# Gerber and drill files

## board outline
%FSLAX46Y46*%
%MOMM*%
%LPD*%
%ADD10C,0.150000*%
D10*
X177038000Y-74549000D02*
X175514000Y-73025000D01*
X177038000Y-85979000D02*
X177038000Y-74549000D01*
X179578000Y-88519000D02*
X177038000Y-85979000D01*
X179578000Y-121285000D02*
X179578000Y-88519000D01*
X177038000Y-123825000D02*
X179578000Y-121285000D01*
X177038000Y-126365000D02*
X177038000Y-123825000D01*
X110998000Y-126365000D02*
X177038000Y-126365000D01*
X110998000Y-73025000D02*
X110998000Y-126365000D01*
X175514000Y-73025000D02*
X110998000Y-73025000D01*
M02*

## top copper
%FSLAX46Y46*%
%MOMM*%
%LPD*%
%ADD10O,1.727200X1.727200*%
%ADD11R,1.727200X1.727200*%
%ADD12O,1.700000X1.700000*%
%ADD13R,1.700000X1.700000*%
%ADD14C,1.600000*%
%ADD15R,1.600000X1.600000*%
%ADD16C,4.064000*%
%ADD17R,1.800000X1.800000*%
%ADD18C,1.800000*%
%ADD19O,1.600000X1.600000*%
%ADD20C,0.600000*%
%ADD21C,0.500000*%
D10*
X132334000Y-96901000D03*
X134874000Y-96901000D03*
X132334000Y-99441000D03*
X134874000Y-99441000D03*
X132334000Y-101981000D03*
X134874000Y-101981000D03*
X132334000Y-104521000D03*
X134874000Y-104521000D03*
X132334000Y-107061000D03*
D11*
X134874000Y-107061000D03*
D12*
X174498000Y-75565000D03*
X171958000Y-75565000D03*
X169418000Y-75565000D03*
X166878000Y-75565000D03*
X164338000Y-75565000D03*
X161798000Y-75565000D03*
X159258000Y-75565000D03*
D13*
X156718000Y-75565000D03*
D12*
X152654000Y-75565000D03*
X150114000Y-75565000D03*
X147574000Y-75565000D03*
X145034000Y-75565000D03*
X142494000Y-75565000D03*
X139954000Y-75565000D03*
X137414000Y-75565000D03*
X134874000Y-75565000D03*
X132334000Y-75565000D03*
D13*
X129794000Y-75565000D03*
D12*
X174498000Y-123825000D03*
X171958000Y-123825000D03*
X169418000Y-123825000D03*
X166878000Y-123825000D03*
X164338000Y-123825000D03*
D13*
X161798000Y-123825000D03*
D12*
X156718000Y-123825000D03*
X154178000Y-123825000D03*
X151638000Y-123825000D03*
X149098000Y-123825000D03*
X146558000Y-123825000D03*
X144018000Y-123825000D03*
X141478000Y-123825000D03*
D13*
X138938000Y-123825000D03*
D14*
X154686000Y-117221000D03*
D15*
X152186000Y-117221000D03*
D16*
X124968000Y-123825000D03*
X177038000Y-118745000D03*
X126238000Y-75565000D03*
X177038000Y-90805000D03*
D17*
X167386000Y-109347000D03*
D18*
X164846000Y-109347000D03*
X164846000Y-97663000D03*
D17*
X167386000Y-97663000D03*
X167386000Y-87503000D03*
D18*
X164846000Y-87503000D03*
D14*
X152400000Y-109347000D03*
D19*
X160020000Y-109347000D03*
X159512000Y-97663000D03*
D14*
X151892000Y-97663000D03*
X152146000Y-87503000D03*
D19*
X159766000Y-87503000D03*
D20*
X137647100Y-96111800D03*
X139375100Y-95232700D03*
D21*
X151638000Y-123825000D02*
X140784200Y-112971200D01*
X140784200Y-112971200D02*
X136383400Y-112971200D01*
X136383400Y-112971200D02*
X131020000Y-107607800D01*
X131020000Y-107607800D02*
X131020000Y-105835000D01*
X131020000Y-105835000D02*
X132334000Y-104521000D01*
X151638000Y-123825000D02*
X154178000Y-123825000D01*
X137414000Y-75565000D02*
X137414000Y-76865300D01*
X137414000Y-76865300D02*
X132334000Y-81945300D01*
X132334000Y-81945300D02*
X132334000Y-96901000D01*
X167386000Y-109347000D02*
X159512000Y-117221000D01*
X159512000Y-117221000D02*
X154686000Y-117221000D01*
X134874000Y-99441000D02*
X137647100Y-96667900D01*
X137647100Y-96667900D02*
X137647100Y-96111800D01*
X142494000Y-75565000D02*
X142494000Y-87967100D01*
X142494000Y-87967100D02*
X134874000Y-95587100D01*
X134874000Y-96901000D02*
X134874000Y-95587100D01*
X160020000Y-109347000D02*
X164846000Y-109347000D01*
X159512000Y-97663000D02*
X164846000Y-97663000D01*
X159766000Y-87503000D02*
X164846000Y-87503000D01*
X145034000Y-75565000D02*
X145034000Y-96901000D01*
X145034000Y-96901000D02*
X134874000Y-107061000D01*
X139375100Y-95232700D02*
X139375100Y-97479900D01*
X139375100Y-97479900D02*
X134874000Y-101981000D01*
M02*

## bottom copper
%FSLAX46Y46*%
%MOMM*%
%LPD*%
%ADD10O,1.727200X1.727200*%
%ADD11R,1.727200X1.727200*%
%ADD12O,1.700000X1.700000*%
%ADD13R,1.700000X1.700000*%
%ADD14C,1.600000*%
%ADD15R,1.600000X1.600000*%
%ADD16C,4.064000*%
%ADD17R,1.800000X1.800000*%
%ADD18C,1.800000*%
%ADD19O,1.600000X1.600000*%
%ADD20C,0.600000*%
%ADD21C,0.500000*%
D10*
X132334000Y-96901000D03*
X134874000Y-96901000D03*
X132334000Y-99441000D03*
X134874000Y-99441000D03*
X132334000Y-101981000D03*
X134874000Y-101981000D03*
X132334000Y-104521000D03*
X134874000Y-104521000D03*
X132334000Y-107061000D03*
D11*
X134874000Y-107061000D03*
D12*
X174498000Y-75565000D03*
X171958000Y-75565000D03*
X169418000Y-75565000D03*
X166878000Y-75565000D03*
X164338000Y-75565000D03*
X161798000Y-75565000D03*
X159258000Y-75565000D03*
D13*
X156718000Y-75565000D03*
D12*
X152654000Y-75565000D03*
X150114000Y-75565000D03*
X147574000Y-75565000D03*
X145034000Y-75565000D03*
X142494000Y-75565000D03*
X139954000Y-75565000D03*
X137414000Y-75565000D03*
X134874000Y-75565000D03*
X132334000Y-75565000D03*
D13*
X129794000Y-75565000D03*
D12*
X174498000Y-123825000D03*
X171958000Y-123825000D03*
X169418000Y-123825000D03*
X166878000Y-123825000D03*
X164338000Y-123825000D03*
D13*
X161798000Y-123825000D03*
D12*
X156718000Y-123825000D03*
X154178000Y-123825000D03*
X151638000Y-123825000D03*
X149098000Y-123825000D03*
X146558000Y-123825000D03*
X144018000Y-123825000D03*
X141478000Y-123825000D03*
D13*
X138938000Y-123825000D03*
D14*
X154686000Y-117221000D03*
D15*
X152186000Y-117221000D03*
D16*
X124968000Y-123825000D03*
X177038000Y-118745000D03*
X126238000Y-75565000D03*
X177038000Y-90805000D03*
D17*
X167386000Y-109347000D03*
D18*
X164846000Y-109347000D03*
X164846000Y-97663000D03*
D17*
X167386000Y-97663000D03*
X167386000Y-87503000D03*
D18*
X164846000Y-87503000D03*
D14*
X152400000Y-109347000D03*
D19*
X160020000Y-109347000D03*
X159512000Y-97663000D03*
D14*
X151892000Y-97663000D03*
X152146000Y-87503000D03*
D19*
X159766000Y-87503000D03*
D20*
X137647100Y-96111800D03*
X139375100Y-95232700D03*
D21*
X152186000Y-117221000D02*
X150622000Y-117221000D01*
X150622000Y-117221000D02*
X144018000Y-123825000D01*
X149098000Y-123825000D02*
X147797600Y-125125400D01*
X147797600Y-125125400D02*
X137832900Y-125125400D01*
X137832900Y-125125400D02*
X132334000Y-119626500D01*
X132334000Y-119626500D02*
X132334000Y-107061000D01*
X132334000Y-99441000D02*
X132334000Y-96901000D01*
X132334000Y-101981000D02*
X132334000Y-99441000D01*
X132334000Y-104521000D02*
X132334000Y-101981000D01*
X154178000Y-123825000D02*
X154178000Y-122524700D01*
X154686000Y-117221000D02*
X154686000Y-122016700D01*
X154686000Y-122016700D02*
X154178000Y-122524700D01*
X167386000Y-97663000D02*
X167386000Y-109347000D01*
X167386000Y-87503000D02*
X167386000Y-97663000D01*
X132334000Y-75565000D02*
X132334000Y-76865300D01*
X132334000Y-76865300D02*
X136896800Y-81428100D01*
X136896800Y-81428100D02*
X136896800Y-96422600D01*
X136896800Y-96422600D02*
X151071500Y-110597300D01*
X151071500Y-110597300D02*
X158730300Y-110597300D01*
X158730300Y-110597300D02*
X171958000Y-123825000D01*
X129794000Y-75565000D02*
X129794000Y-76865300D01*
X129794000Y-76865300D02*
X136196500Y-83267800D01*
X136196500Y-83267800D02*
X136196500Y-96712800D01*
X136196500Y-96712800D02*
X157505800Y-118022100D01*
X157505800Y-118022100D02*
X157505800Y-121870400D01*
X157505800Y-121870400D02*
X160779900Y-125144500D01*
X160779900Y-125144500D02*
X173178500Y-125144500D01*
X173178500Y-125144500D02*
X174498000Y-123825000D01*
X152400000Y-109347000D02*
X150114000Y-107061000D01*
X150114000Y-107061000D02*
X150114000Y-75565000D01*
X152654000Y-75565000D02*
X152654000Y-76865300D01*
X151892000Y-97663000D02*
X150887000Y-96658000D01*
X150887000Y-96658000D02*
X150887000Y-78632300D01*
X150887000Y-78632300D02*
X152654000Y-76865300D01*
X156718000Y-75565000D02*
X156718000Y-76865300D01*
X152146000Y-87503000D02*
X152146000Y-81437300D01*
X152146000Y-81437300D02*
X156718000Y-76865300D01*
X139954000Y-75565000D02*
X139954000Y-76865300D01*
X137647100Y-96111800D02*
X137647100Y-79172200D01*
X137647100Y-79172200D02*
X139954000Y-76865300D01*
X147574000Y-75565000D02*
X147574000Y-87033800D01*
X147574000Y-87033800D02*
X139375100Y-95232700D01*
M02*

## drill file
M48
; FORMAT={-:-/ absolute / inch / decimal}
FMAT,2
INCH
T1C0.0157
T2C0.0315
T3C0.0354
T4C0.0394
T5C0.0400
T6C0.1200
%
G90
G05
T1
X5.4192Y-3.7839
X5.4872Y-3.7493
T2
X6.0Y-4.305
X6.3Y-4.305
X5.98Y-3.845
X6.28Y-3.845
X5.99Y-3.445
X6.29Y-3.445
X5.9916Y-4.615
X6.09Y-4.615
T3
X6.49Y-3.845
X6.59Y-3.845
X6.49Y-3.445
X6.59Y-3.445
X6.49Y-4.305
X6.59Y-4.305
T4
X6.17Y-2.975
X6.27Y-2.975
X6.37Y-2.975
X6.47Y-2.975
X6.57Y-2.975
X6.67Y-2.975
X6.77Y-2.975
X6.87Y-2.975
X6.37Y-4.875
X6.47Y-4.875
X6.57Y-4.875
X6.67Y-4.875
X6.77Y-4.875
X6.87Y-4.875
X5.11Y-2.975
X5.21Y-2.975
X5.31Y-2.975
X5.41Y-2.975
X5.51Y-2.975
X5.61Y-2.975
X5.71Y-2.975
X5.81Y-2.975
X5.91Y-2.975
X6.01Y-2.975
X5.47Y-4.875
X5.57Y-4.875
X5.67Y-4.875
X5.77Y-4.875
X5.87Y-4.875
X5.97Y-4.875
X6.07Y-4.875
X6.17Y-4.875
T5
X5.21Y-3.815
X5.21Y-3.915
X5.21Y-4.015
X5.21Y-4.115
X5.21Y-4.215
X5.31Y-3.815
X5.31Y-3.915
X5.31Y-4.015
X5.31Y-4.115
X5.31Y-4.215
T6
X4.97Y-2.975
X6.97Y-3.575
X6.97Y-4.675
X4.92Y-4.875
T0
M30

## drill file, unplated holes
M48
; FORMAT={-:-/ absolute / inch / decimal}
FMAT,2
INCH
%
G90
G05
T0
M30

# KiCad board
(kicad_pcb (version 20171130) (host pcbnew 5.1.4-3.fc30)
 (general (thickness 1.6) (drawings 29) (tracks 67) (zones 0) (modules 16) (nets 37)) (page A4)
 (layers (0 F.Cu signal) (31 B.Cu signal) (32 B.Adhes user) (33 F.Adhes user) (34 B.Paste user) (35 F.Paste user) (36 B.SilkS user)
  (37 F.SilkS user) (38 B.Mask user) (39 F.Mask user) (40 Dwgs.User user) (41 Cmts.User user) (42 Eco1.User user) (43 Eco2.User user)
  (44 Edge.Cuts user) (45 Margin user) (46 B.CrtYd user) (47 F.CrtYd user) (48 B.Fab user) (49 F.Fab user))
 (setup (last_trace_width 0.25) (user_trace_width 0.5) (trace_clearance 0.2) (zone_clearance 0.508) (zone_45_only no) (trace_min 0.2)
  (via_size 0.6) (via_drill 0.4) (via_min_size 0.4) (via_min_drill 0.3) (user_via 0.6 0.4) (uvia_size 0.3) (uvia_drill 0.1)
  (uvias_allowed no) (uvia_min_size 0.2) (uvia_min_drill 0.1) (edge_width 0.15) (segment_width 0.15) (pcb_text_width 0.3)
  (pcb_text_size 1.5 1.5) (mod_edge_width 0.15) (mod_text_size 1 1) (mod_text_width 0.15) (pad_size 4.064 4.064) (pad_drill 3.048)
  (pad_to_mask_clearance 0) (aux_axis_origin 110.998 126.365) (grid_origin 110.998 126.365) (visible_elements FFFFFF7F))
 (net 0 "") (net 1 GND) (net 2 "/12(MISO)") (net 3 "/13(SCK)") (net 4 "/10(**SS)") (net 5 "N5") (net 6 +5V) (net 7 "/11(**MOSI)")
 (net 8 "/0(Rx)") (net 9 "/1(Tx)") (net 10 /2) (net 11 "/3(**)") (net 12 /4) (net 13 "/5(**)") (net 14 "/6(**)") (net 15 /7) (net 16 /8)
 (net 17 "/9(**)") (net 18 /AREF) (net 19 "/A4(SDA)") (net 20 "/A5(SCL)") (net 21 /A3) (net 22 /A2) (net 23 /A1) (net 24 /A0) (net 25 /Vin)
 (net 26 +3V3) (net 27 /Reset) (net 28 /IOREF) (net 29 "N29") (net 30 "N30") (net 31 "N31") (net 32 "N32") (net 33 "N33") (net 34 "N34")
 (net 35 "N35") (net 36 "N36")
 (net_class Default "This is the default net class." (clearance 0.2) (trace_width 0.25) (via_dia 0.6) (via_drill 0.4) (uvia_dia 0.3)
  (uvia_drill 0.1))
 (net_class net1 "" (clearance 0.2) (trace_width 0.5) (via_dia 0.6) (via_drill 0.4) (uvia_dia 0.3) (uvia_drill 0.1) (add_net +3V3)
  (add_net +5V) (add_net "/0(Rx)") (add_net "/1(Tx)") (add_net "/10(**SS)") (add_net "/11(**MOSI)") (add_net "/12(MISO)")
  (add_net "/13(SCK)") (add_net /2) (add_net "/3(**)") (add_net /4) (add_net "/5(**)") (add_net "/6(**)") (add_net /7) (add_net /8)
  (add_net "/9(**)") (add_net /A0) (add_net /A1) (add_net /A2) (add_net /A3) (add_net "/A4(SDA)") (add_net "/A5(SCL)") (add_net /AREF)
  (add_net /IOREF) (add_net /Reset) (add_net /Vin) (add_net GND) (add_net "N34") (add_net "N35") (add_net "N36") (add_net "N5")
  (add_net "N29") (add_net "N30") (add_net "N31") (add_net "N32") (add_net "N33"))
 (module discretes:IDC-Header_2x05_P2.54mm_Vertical (layer F.Cu) (at 134.874 107.061 180)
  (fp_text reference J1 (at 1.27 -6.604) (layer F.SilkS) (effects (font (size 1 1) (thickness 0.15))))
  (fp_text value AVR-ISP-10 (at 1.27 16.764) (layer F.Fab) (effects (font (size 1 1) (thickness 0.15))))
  (pad 10 thru_hole oval (at 2.54 10.16 180) (size 1.7272 1.7272) (drill 1.016) (layers *.Cu *.Mask) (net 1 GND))
  (pad 9 thru_hole oval (at 0 10.16 180) (size 1.7272 1.7272) (drill 1.016) (layers *.Cu *.Mask) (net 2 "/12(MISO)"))
  (pad 8 thru_hole oval (at 2.54 7.62 180) (size 1.7272 1.7272) (drill 1.016) (layers *.Cu *.Mask) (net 1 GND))
  (pad 7 thru_hole oval (at 0 7.62 180) (size 1.7272 1.7272) (drill 1.016) (layers *.Cu *.Mask) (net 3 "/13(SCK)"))
  (pad 6 thru_hole oval (at 2.54 5.08 180) (size 1.7272 1.7272) (drill 1.016) (layers *.Cu *.Mask) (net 1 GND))
  (pad 5 thru_hole oval (at 0 5.08 180) (size 1.7272 1.7272) (drill 1.016) (layers *.Cu *.Mask) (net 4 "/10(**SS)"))
  (pad 4 thru_hole oval (at 2.54 2.54 180) (size 1.7272 1.7272) (drill 1.016) (layers *.Cu *.Mask) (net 1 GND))
  (pad 3 thru_hole oval (at 0 2.54 180) (size 1.7272 1.7272) (drill 1.016) (layers *.Cu *.Mask) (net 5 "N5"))
  (pad 2 thru_hole oval (at 2.54 0 180) (size 1.7272 1.7272) (drill 1.016) (layers *.Cu *.Mask) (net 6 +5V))
  (pad 1 thru_hole rect (at 0 0 180) (size 1.7272 1.7272) (drill 1.016) (layers *.Cu *.Mask) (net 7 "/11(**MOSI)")))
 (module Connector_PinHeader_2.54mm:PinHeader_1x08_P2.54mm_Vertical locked (layer B.Cu) (at 156.718 75.565 270)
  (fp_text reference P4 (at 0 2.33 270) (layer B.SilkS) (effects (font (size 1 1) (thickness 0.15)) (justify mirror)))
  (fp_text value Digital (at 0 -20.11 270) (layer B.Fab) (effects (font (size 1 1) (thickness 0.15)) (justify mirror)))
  (pad 8 thru_hole oval (at 0 -17.78 270) (size 1.7 1.7) (drill 1) (layers *.Cu *.Mask) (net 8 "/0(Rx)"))
  (pad 7 thru_hole oval (at 0 -15.24 270) (size 1.7 1.7) (drill 1) (layers *.Cu *.Mask) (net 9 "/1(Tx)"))
  (pad 6 thru_hole oval (at 0 -12.7 270) (size 1.7 1.7) (drill 1) (layers *.Cu *.Mask) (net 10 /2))
  (pad 5 thru_hole oval (at 0 -10.16 270) (size 1.7 1.7) (drill 1) (layers *.Cu *.Mask) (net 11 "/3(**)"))
  (pad 4 thru_hole oval (at 0 -7.62 270) (size 1.7 1.7) (drill 1) (layers *.Cu *.Mask) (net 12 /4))
  (pad 3 thru_hole oval (at 0 -5.08 270) (size 1.7 1.7) (drill 1) (layers *.Cu *.Mask) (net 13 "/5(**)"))
  (pad 2 thru_hole oval (at 0 -2.54 270) (size 1.7 1.7) (drill 1) (layers *.Cu *.Mask) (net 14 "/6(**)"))
  (pad 1 thru_hole rect (at 0 0 270) (size 1.7 1.7) (drill 1) (layers *.Cu *.Mask) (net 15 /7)))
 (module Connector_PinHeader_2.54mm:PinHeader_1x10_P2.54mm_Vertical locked (layer B.Cu) (at 129.794 75.565 270)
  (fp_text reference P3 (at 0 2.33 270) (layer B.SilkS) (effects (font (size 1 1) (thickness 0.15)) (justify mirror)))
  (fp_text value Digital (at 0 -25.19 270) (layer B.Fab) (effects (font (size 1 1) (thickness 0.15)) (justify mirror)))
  (pad 10 thru_hole oval (at 0 -22.86 270) (size 1.7 1.7) (drill 1) (layers *.Cu *.Mask) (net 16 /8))
  (pad 9 thru_hole oval (at 0 -20.32 270) (size 1.7 1.7) (drill 1) (layers *.Cu *.Mask) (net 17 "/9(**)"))
  (pad 8 thru_hole oval (at 0 -17.78 270) (size 1.7 1.7) (drill 1) (layers *.Cu *.Mask) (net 4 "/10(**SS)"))
  (pad 7 thru_hole oval (at 0 -15.24 270) (size 1.7 1.7) (drill 1) (layers *.Cu *.Mask) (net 7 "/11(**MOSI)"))
  (pad 6 thru_hole oval (at 0 -12.7 270) (size 1.7 1.7) (drill 1) (layers *.Cu *.Mask) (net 2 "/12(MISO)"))
  (pad 5 thru_hole oval (at 0 -10.16 270) (size 1.7 1.7) (drill 1) (layers *.Cu *.Mask) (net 3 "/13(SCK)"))
  (pad 4 thru_hole oval (at 0 -7.62 270) (size 1.7 1.7) (drill 1) (layers *.Cu *.Mask) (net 1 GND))
  (pad 3 thru_hole oval (at 0 -5.08 270) (size 1.7 1.7) (drill 1) (layers *.Cu *.Mask) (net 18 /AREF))
  (pad 2 thru_hole oval (at 0 -2.54 270) (size 1.7 1.7) (drill 1) (layers *.Cu *.Mask) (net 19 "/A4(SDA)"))
  (pad 1 thru_hole rect (at 0 0 270) (size 1.7 1.7) (drill 1) (layers *.Cu *.Mask) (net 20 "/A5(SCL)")))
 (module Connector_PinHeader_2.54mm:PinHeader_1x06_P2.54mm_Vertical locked (layer B.Cu) (at 161.798 123.825 270)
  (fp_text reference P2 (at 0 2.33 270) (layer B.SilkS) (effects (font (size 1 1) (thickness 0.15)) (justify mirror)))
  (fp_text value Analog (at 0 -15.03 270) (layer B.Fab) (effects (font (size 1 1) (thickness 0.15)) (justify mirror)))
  (pad 6 thru_hole oval (at 0 -12.7 270) (size 1.7 1.7) (drill 1) (layers *.Cu *.Mask) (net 20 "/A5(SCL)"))
  (pad 5 thru_hole oval (at 0 -10.16 270) (size 1.7 1.7) (drill 1) (layers *.Cu *.Mask) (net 19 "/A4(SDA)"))
  (pad 4 thru_hole oval (at 0 -7.62 270) (size 1.7 1.7) (drill 1) (layers *.Cu *.Mask) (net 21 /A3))
  (pad 3 thru_hole oval (at 0 -5.08 270) (size 1.7 1.7) (drill 1) (layers *.Cu *.Mask) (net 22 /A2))
  (pad 2 thru_hole oval (at 0 -2.54 270) (size 1.7 1.7) (drill 1) (layers *.Cu *.Mask) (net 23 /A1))
  (pad 1 thru_hole rect (at 0 0 270) (size 1.7 1.7) (drill 1) (layers *.Cu *.Mask) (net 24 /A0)))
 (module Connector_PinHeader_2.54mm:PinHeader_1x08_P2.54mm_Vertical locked (layer B.Cu) (at 138.938 123.825 270)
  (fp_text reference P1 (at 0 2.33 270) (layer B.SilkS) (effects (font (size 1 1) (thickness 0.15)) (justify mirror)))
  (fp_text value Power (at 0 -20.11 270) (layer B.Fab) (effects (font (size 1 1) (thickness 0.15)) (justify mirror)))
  (pad 8 thru_hole oval (at 0 -17.78 270) (size 1.7 1.7) (drill 1) (layers *.Cu *.Mask) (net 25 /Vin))
  (pad 7 thru_hole oval (at 0 -15.24 270) (size 1.7 1.7) (drill 1) (layers *.Cu *.Mask) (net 1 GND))
  (pad 6 thru_hole oval (at 0 -12.7 270) (size 1.7 1.7) (drill 1) (layers *.Cu *.Mask) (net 1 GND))
  (pad 5 thru_hole oval (at 0 -10.16 270) (size 1.7 1.7) (drill 1) (layers *.Cu *.Mask) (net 6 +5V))
  (pad 4 thru_hole oval (at 0 -7.62 270) (size 1.7 1.7) (drill 1) (layers *.Cu *.Mask) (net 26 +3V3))
  (pad 3 thru_hole oval (at 0 -5.08 270) (size 1.7 1.7) (drill 1) (layers *.Cu *.Mask) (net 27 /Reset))
  (pad 2 thru_hole oval (at 0 -2.54 270) (size 1.7 1.7) (drill 1) (layers *.Cu *.Mask) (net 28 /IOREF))
  (pad 1 thru_hole rect (at 0 0 270) (size 1.7 1.7) (drill 1) (layers *.Cu *.Mask) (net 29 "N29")))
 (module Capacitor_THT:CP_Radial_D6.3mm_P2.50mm (layer F.Cu) (at 152.186 117.221)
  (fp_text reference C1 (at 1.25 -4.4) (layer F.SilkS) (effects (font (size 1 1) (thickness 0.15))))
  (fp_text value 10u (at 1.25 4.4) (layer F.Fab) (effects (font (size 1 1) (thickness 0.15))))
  (pad 2 thru_hole circle (at 2.5 0) (size 1.6 1.6) (drill 0.8) (layers *.Cu *.Mask) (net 1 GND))
  (pad 1 thru_hole rect (at 0 0) (size 1.6 1.6) (drill 0.8) (layers *.Cu *.Mask) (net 27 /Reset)))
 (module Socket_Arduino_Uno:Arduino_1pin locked (layer F.Cu) (at 124.968 123.825)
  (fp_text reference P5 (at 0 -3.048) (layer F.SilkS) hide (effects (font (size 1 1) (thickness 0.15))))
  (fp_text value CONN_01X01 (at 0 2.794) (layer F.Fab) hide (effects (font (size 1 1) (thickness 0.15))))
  (pad 1 thru_hole circle (at 0 0) (size 4.064 4.064) (drill 3.048) (layers *.Cu *.Mask F.SilkS) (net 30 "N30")))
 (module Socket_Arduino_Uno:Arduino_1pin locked (layer F.Cu) (at 177.038 118.745)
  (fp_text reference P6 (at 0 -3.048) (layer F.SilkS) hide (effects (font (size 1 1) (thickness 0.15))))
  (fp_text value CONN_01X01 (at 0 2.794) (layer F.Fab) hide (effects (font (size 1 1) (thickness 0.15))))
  (pad 1 thru_hole circle (at 0 0) (size 4.064 4.064) (drill 3.048) (layers *.Cu *.Mask F.SilkS) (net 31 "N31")))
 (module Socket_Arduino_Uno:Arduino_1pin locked (layer F.Cu) (at 126.238 75.565)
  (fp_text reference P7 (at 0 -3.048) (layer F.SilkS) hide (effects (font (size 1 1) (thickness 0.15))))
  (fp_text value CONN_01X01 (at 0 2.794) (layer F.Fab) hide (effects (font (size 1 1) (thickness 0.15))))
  (pad 1 thru_hole circle (at 0 0) (size 4.064 4.064) (drill 3.048) (layers *.Cu *.Mask F.SilkS) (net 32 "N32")))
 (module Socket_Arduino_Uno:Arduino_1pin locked (layer F.Cu) (at 177.038 90.805)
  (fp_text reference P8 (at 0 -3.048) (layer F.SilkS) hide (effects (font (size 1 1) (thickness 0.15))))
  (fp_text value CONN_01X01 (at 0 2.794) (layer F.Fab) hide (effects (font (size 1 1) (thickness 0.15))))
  (pad 1 thru_hole circle (at 0 0) (size 4.064 4.064) (drill 3.048) (layers *.Cu *.Mask F.SilkS) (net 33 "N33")))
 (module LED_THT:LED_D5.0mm (layer F.Cu) (at 167.386 109.347 180)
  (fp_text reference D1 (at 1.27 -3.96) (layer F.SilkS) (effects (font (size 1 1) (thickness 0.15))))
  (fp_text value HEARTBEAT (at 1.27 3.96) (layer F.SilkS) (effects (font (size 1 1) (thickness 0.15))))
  (pad 1 thru_hole rect (at 0 0 180) (size 1.8 1.8) (drill 0.9) (layers *.Cu *.Mask) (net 1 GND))
  (pad 2 thru_hole circle (at 2.54 0 180) (size 1.8 1.8) (drill 0.9) (layers *.Cu *.Mask) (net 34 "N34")))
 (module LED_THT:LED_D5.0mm (layer F.Cu) (at 167.386 97.663 180)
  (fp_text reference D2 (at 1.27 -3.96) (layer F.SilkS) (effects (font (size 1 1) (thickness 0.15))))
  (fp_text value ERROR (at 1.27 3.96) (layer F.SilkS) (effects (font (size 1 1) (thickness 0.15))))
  (pad 2 thru_hole circle (at 2.54 0 180) (size 1.8 1.8) (drill 0.9) (layers *.Cu *.Mask) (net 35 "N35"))
  (pad 1 thru_hole rect (at 0 0 180) (size 1.8 1.8) (drill 0.9) (layers *.Cu *.Mask) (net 1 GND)))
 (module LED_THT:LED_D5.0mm (layer F.Cu) (at 167.386 87.503 180)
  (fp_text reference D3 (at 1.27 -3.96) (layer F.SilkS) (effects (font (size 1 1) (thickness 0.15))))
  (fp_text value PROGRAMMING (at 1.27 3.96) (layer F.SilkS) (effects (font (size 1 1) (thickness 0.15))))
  (pad 1 thru_hole rect (at 0 0 180) (size 1.8 1.8) (drill 0.9) (layers *.Cu *.Mask) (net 1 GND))
  (pad 2 thru_hole circle (at 2.54 0 180) (size 1.8 1.8) (drill 0.9) (layers *.Cu *.Mask) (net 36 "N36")))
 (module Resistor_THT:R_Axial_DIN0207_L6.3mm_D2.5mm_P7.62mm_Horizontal (layer F.Cu) (at 152.4 109.347)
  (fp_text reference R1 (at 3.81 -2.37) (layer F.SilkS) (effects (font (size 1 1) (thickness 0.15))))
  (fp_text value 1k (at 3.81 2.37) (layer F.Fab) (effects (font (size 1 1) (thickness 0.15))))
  (pad 1 thru_hole circle (at 0 0) (size 1.6 1.6) (drill 0.8) (layers *.Cu *.Mask) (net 17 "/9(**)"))
  (pad 2 thru_hole oval (at 7.62 0) (size 1.6 1.6) (drill 0.8) (layers *.Cu *.Mask) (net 34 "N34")))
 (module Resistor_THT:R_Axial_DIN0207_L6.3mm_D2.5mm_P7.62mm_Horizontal (layer F.Cu) (at 151.892 97.663)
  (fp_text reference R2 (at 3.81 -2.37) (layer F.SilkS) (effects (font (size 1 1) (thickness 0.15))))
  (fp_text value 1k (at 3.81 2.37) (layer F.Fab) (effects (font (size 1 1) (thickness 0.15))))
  (pad 2 thru_hole oval (at 7.62 0) (size 1.6 1.6) (drill 0.8) (layers *.Cu *.Mask) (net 35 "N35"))
  (pad 1 thru_hole circle (at 0 0) (size 1.6 1.6) (drill 0.8) (layers *.Cu *.Mask) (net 16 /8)))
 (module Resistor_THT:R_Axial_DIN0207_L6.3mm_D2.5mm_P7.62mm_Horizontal (layer F.Cu) (at 152.146 87.503)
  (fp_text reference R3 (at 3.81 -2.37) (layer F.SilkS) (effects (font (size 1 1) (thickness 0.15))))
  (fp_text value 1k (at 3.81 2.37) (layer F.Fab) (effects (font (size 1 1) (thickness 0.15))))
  (pad 1 thru_hole circle (at 0 0) (size 1.6 1.6) (drill 0.8) (layers *.Cu *.Mask) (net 15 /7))
  (pad 2 thru_hole oval (at 7.62 0) (size 1.6 1.6) (drill 0.8) (layers *.Cu *.Mask) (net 36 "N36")))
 (gr_line (start 177.038 74.549) (end 175.514 73.025) (angle 90) (layer Edge.Cuts) (width 0.15))
 (gr_line (start 177.038 85.979) (end 177.038 74.549) (angle 90) (layer Edge.Cuts) (width 0.15))
 (gr_line (start 179.578 88.519) (end 177.038 85.979) (angle 90) (layer Edge.Cuts) (width 0.15))
 (gr_line (start 179.578 121.285) (end 179.578 88.519) (angle 90) (layer Edge.Cuts) (width 0.15))
 (gr_line (start 177.038 123.825) (end 179.578 121.285) (angle 90) (layer Edge.Cuts) (width 0.15))
 (gr_line (start 177.038 126.365) (end 177.038 123.825) (angle 90) (layer Edge.Cuts) (width 0.15))
 (gr_line (start 110.998 126.365) (end 177.038 126.365) (angle 90) (layer Edge.Cuts) (width 0.15))
 (gr_line (start 110.998 73.025) (end 110.998 126.365) (angle 90) (layer Edge.Cuts) (width 0.15))
 (gr_line (start 175.514 73.025) (end 110.998 73.025) (angle 90) (layer Edge.Cuts) (width 0.15))
 (segment (start 152.186 117.221) (end 150.622 117.221) (width 0.5) (layer B.Cu) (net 27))
 (segment (start 150.622 117.221) (end 144.018 123.825) (width 0.5) (layer B.Cu) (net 27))
 (segment (start 149.098 123.825) (end 147.7976 125.1254) (width 0.5) (layer B.Cu) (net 6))
 (segment (start 147.7976 125.1254) (end 137.8329 125.1254) (width 0.5) (layer B.Cu) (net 6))
 (segment (start 137.8329 125.1254) (end 132.334 119.6265) (width 0.5) (layer B.Cu) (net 6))
 (segment (start 132.334 119.6265) (end 132.334 107.061) (width 0.5) (layer B.Cu) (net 6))
 (segment (start 151.638 123.825) (end 140.7842 112.9712) (width 0.5) (layer F.Cu) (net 1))
 (segment (start 140.7842 112.9712) (end 136.3834 112.9712) (width 0.5) (layer F.Cu) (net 1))
 (segment (start 136.3834 112.9712) (end 131.02 107.6078) (width 0.5) (layer F.Cu) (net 1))
 (segment (start 131.02 107.6078) (end 131.02 105.835) (width 0.5) (layer F.Cu) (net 1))
 (segment (start 131.02 105.835) (end 132.334 104.521) (width 0.5) (layer F.Cu) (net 1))
 (segment (start 151.638 123.825) (end 154.178 123.825) (width 0.5) (layer F.Cu) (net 1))
 (segment (start 137.414 75.565) (end 137.414 76.8653) (width 0.5) (layer F.Cu) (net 1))
 (segment (start 137.414 76.8653) (end 132.334 81.9453) (width 0.5) (layer F.Cu) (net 1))
 (segment (start 132.334 81.9453) (end 132.334 96.901) (width 0.5) (layer F.Cu) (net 1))
 (segment (start 132.334 99.441) (end 132.334 96.901) (width 0.5) (layer B.Cu) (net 1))
 (segment (start 132.334 101.981) (end 132.334 99.441) (width 0.5) (layer B.Cu) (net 1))
 (segment (start 132.334 104.521) (end 132.334 101.981) (width 0.5) (layer B.Cu) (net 1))
 (segment (start 154.178 123.825) (end 154.178 122.5247) (width 0.5) (layer B.Cu) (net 1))
 (segment (start 154.686 117.221) (end 154.686 122.0167) (width 0.5) (layer B.Cu) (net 1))
 (segment (start 154.686 122.0167) (end 154.178 122.5247) (width 0.5) (layer B.Cu) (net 1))
 (segment (start 167.386 109.347) (end 159.512 117.221) (width 0.5) (layer F.Cu) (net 1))
 (segment (start 159.512 117.221) (end 154.686 117.221) (width 0.5) (layer F.Cu) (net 1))
 (segment (start 167.386 97.663) (end 167.386 109.347) (width 0.5) (layer B.Cu) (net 1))
 (segment (start 167.386 87.503) (end 167.386 97.663) (width 0.5) (layer B.Cu) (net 1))
 (segment (start 132.334 75.565) (end 132.334 76.8653) (width 0.5) (layer B.Cu) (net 19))
 (segment (start 132.334 76.8653) (end 136.8968 81.4281) (width 0.5) (layer B.Cu) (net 19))
 (segment (start 136.8968 81.4281) (end 136.8968 96.4226) (width 0.5) (layer B.Cu) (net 19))
 (segment (start 136.8968 96.4226) (end 151.0715 110.5973) (width 0.5) (layer B.Cu) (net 19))
 (segment (start 151.0715 110.5973) (end 158.7303 110.5973) (width 0.5) (layer B.Cu) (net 19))
 (segment (start 158.7303 110.5973) (end 171.958 123.825) (width 0.5) (layer B.Cu) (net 19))
 (segment (start 129.794 75.565) (end 129.794 76.8653) (width 0.5) (layer B.Cu) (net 20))
 (segment (start 129.794 76.8653) (end 136.1965 83.2678) (width 0.5) (layer B.Cu) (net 20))
 (segment (start 136.1965 83.2678) (end 136.1965 96.7128) (width 0.5) (layer B.Cu) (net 20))
 (segment (start 136.1965 96.7128) (end 157.5058 118.0221) (width 0.5) (layer B.Cu) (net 20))
 (segment (start 157.5058 118.0221) (end 157.5058 121.8704) (width 0.5) (layer B.Cu) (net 20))
 (segment (start 157.5058 121.8704) (end 160.7799 125.1445) (width 0.5) (layer B.Cu) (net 20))
 (segment (start 160.7799 125.1445) (end 173.1785 125.1445) (width 0.5) (layer B.Cu) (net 20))
 (segment (start 173.1785 125.1445) (end 174.498 123.825) (width 0.5) (layer B.Cu) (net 20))
 (segment (start 152.4 109.347) (end 150.114 107.061) (width 0.5) (layer B.Cu) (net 17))
 (segment (start 150.114 107.061) (end 150.114 75.565) (width 0.5) (layer B.Cu) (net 17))
 (segment (start 152.654 75.565) (end 152.654 76.8653) (width 0.5) (layer B.Cu) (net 16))
 (segment (start 151.892 97.663) (end 150.887 96.658) (width 0.5) (layer B.Cu) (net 16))
 (segment (start 150.887 96.658) (end 150.887 78.6323) (width 0.5) (layer B.Cu) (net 16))
 (segment (start 150.887 78.6323) (end 152.654 76.8653) (width 0.5) (layer B.Cu) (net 16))
 (segment (start 156.718 75.565) (end 156.718 76.8653) (width 0.5) (layer B.Cu) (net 15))
 (segment (start 152.146 87.503) (end 152.146 81.4373) (width 0.5) (layer B.Cu) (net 15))
 (segment (start 152.146 81.4373) (end 156.718 76.8653) (width 0.5) (layer B.Cu) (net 15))
 (segment (start 139.954 75.565) (end 139.954 76.8653) (width 0.5) (layer B.Cu) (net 3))
 (segment (start 137.6471 96.1118) (end 137.6471 79.1722) (width 0.5) (layer B.Cu) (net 3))
 (segment (start 137.6471 79.1722) (end 139.954 76.8653) (width 0.5) (layer B.Cu) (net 3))
 (segment (start 134.874 99.441) (end 137.6471 96.6679) (width 0.5) (layer F.Cu) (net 3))
 (segment (start 137.6471 96.6679) (end 137.6471 96.1118) (width 0.5) (layer F.Cu) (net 3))
 (via (at 137.6471 96.1118) (size 0.6) (layers F.Cu B.Cu) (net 3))
 (segment (start 142.494 75.565) (end 142.494 87.9671) (width 0.5) (layer F.Cu) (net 2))
 (segment (start 142.494 87.9671) (end 134.874 95.5871) (width 0.5) (layer F.Cu) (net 2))
 (segment (start 134.874 96.901) (end 134.874 95.5871) (width 0.5) (layer F.Cu) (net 2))
 (segment (start 160.02 109.347) (end 164.846 109.347) (width 0.5) (layer F.Cu) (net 34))
 (segment (start 159.512 97.663) (end 164.846 97.663) (width 0.5) (layer F.Cu) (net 35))
 (segment (start 159.766 87.503) (end 164.846 87.503) (width 0.5) (layer F.Cu) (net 36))
 (segment (start 145.034 75.565) (end 145.034 96.901) (width 0.5) (layer F.Cu) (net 7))
 (segment (start 145.034 96.901) (end 134.874 107.061) (width 0.5) (layer F.Cu) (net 7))
 (segment (start 139.3751 95.2327) (end 139.3751 97.4799) (width 0.5) (layer F.Cu) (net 4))
 (segment (start 139.3751 97.4799) (end 134.874 101.981) (width 0.5) (layer F.Cu) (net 4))
 (segment (start 147.574 75.565) (end 147.574 87.0338) (width 0.5) (layer B.Cu) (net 4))
 (segment (start 147.574 87.0338) (end 139.3751 95.2327) (width 0.5) (layer B.Cu) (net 4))
 (via (at 139.3751 95.2327) (size 0.6) (layers F.Cu B.Cu) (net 4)))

